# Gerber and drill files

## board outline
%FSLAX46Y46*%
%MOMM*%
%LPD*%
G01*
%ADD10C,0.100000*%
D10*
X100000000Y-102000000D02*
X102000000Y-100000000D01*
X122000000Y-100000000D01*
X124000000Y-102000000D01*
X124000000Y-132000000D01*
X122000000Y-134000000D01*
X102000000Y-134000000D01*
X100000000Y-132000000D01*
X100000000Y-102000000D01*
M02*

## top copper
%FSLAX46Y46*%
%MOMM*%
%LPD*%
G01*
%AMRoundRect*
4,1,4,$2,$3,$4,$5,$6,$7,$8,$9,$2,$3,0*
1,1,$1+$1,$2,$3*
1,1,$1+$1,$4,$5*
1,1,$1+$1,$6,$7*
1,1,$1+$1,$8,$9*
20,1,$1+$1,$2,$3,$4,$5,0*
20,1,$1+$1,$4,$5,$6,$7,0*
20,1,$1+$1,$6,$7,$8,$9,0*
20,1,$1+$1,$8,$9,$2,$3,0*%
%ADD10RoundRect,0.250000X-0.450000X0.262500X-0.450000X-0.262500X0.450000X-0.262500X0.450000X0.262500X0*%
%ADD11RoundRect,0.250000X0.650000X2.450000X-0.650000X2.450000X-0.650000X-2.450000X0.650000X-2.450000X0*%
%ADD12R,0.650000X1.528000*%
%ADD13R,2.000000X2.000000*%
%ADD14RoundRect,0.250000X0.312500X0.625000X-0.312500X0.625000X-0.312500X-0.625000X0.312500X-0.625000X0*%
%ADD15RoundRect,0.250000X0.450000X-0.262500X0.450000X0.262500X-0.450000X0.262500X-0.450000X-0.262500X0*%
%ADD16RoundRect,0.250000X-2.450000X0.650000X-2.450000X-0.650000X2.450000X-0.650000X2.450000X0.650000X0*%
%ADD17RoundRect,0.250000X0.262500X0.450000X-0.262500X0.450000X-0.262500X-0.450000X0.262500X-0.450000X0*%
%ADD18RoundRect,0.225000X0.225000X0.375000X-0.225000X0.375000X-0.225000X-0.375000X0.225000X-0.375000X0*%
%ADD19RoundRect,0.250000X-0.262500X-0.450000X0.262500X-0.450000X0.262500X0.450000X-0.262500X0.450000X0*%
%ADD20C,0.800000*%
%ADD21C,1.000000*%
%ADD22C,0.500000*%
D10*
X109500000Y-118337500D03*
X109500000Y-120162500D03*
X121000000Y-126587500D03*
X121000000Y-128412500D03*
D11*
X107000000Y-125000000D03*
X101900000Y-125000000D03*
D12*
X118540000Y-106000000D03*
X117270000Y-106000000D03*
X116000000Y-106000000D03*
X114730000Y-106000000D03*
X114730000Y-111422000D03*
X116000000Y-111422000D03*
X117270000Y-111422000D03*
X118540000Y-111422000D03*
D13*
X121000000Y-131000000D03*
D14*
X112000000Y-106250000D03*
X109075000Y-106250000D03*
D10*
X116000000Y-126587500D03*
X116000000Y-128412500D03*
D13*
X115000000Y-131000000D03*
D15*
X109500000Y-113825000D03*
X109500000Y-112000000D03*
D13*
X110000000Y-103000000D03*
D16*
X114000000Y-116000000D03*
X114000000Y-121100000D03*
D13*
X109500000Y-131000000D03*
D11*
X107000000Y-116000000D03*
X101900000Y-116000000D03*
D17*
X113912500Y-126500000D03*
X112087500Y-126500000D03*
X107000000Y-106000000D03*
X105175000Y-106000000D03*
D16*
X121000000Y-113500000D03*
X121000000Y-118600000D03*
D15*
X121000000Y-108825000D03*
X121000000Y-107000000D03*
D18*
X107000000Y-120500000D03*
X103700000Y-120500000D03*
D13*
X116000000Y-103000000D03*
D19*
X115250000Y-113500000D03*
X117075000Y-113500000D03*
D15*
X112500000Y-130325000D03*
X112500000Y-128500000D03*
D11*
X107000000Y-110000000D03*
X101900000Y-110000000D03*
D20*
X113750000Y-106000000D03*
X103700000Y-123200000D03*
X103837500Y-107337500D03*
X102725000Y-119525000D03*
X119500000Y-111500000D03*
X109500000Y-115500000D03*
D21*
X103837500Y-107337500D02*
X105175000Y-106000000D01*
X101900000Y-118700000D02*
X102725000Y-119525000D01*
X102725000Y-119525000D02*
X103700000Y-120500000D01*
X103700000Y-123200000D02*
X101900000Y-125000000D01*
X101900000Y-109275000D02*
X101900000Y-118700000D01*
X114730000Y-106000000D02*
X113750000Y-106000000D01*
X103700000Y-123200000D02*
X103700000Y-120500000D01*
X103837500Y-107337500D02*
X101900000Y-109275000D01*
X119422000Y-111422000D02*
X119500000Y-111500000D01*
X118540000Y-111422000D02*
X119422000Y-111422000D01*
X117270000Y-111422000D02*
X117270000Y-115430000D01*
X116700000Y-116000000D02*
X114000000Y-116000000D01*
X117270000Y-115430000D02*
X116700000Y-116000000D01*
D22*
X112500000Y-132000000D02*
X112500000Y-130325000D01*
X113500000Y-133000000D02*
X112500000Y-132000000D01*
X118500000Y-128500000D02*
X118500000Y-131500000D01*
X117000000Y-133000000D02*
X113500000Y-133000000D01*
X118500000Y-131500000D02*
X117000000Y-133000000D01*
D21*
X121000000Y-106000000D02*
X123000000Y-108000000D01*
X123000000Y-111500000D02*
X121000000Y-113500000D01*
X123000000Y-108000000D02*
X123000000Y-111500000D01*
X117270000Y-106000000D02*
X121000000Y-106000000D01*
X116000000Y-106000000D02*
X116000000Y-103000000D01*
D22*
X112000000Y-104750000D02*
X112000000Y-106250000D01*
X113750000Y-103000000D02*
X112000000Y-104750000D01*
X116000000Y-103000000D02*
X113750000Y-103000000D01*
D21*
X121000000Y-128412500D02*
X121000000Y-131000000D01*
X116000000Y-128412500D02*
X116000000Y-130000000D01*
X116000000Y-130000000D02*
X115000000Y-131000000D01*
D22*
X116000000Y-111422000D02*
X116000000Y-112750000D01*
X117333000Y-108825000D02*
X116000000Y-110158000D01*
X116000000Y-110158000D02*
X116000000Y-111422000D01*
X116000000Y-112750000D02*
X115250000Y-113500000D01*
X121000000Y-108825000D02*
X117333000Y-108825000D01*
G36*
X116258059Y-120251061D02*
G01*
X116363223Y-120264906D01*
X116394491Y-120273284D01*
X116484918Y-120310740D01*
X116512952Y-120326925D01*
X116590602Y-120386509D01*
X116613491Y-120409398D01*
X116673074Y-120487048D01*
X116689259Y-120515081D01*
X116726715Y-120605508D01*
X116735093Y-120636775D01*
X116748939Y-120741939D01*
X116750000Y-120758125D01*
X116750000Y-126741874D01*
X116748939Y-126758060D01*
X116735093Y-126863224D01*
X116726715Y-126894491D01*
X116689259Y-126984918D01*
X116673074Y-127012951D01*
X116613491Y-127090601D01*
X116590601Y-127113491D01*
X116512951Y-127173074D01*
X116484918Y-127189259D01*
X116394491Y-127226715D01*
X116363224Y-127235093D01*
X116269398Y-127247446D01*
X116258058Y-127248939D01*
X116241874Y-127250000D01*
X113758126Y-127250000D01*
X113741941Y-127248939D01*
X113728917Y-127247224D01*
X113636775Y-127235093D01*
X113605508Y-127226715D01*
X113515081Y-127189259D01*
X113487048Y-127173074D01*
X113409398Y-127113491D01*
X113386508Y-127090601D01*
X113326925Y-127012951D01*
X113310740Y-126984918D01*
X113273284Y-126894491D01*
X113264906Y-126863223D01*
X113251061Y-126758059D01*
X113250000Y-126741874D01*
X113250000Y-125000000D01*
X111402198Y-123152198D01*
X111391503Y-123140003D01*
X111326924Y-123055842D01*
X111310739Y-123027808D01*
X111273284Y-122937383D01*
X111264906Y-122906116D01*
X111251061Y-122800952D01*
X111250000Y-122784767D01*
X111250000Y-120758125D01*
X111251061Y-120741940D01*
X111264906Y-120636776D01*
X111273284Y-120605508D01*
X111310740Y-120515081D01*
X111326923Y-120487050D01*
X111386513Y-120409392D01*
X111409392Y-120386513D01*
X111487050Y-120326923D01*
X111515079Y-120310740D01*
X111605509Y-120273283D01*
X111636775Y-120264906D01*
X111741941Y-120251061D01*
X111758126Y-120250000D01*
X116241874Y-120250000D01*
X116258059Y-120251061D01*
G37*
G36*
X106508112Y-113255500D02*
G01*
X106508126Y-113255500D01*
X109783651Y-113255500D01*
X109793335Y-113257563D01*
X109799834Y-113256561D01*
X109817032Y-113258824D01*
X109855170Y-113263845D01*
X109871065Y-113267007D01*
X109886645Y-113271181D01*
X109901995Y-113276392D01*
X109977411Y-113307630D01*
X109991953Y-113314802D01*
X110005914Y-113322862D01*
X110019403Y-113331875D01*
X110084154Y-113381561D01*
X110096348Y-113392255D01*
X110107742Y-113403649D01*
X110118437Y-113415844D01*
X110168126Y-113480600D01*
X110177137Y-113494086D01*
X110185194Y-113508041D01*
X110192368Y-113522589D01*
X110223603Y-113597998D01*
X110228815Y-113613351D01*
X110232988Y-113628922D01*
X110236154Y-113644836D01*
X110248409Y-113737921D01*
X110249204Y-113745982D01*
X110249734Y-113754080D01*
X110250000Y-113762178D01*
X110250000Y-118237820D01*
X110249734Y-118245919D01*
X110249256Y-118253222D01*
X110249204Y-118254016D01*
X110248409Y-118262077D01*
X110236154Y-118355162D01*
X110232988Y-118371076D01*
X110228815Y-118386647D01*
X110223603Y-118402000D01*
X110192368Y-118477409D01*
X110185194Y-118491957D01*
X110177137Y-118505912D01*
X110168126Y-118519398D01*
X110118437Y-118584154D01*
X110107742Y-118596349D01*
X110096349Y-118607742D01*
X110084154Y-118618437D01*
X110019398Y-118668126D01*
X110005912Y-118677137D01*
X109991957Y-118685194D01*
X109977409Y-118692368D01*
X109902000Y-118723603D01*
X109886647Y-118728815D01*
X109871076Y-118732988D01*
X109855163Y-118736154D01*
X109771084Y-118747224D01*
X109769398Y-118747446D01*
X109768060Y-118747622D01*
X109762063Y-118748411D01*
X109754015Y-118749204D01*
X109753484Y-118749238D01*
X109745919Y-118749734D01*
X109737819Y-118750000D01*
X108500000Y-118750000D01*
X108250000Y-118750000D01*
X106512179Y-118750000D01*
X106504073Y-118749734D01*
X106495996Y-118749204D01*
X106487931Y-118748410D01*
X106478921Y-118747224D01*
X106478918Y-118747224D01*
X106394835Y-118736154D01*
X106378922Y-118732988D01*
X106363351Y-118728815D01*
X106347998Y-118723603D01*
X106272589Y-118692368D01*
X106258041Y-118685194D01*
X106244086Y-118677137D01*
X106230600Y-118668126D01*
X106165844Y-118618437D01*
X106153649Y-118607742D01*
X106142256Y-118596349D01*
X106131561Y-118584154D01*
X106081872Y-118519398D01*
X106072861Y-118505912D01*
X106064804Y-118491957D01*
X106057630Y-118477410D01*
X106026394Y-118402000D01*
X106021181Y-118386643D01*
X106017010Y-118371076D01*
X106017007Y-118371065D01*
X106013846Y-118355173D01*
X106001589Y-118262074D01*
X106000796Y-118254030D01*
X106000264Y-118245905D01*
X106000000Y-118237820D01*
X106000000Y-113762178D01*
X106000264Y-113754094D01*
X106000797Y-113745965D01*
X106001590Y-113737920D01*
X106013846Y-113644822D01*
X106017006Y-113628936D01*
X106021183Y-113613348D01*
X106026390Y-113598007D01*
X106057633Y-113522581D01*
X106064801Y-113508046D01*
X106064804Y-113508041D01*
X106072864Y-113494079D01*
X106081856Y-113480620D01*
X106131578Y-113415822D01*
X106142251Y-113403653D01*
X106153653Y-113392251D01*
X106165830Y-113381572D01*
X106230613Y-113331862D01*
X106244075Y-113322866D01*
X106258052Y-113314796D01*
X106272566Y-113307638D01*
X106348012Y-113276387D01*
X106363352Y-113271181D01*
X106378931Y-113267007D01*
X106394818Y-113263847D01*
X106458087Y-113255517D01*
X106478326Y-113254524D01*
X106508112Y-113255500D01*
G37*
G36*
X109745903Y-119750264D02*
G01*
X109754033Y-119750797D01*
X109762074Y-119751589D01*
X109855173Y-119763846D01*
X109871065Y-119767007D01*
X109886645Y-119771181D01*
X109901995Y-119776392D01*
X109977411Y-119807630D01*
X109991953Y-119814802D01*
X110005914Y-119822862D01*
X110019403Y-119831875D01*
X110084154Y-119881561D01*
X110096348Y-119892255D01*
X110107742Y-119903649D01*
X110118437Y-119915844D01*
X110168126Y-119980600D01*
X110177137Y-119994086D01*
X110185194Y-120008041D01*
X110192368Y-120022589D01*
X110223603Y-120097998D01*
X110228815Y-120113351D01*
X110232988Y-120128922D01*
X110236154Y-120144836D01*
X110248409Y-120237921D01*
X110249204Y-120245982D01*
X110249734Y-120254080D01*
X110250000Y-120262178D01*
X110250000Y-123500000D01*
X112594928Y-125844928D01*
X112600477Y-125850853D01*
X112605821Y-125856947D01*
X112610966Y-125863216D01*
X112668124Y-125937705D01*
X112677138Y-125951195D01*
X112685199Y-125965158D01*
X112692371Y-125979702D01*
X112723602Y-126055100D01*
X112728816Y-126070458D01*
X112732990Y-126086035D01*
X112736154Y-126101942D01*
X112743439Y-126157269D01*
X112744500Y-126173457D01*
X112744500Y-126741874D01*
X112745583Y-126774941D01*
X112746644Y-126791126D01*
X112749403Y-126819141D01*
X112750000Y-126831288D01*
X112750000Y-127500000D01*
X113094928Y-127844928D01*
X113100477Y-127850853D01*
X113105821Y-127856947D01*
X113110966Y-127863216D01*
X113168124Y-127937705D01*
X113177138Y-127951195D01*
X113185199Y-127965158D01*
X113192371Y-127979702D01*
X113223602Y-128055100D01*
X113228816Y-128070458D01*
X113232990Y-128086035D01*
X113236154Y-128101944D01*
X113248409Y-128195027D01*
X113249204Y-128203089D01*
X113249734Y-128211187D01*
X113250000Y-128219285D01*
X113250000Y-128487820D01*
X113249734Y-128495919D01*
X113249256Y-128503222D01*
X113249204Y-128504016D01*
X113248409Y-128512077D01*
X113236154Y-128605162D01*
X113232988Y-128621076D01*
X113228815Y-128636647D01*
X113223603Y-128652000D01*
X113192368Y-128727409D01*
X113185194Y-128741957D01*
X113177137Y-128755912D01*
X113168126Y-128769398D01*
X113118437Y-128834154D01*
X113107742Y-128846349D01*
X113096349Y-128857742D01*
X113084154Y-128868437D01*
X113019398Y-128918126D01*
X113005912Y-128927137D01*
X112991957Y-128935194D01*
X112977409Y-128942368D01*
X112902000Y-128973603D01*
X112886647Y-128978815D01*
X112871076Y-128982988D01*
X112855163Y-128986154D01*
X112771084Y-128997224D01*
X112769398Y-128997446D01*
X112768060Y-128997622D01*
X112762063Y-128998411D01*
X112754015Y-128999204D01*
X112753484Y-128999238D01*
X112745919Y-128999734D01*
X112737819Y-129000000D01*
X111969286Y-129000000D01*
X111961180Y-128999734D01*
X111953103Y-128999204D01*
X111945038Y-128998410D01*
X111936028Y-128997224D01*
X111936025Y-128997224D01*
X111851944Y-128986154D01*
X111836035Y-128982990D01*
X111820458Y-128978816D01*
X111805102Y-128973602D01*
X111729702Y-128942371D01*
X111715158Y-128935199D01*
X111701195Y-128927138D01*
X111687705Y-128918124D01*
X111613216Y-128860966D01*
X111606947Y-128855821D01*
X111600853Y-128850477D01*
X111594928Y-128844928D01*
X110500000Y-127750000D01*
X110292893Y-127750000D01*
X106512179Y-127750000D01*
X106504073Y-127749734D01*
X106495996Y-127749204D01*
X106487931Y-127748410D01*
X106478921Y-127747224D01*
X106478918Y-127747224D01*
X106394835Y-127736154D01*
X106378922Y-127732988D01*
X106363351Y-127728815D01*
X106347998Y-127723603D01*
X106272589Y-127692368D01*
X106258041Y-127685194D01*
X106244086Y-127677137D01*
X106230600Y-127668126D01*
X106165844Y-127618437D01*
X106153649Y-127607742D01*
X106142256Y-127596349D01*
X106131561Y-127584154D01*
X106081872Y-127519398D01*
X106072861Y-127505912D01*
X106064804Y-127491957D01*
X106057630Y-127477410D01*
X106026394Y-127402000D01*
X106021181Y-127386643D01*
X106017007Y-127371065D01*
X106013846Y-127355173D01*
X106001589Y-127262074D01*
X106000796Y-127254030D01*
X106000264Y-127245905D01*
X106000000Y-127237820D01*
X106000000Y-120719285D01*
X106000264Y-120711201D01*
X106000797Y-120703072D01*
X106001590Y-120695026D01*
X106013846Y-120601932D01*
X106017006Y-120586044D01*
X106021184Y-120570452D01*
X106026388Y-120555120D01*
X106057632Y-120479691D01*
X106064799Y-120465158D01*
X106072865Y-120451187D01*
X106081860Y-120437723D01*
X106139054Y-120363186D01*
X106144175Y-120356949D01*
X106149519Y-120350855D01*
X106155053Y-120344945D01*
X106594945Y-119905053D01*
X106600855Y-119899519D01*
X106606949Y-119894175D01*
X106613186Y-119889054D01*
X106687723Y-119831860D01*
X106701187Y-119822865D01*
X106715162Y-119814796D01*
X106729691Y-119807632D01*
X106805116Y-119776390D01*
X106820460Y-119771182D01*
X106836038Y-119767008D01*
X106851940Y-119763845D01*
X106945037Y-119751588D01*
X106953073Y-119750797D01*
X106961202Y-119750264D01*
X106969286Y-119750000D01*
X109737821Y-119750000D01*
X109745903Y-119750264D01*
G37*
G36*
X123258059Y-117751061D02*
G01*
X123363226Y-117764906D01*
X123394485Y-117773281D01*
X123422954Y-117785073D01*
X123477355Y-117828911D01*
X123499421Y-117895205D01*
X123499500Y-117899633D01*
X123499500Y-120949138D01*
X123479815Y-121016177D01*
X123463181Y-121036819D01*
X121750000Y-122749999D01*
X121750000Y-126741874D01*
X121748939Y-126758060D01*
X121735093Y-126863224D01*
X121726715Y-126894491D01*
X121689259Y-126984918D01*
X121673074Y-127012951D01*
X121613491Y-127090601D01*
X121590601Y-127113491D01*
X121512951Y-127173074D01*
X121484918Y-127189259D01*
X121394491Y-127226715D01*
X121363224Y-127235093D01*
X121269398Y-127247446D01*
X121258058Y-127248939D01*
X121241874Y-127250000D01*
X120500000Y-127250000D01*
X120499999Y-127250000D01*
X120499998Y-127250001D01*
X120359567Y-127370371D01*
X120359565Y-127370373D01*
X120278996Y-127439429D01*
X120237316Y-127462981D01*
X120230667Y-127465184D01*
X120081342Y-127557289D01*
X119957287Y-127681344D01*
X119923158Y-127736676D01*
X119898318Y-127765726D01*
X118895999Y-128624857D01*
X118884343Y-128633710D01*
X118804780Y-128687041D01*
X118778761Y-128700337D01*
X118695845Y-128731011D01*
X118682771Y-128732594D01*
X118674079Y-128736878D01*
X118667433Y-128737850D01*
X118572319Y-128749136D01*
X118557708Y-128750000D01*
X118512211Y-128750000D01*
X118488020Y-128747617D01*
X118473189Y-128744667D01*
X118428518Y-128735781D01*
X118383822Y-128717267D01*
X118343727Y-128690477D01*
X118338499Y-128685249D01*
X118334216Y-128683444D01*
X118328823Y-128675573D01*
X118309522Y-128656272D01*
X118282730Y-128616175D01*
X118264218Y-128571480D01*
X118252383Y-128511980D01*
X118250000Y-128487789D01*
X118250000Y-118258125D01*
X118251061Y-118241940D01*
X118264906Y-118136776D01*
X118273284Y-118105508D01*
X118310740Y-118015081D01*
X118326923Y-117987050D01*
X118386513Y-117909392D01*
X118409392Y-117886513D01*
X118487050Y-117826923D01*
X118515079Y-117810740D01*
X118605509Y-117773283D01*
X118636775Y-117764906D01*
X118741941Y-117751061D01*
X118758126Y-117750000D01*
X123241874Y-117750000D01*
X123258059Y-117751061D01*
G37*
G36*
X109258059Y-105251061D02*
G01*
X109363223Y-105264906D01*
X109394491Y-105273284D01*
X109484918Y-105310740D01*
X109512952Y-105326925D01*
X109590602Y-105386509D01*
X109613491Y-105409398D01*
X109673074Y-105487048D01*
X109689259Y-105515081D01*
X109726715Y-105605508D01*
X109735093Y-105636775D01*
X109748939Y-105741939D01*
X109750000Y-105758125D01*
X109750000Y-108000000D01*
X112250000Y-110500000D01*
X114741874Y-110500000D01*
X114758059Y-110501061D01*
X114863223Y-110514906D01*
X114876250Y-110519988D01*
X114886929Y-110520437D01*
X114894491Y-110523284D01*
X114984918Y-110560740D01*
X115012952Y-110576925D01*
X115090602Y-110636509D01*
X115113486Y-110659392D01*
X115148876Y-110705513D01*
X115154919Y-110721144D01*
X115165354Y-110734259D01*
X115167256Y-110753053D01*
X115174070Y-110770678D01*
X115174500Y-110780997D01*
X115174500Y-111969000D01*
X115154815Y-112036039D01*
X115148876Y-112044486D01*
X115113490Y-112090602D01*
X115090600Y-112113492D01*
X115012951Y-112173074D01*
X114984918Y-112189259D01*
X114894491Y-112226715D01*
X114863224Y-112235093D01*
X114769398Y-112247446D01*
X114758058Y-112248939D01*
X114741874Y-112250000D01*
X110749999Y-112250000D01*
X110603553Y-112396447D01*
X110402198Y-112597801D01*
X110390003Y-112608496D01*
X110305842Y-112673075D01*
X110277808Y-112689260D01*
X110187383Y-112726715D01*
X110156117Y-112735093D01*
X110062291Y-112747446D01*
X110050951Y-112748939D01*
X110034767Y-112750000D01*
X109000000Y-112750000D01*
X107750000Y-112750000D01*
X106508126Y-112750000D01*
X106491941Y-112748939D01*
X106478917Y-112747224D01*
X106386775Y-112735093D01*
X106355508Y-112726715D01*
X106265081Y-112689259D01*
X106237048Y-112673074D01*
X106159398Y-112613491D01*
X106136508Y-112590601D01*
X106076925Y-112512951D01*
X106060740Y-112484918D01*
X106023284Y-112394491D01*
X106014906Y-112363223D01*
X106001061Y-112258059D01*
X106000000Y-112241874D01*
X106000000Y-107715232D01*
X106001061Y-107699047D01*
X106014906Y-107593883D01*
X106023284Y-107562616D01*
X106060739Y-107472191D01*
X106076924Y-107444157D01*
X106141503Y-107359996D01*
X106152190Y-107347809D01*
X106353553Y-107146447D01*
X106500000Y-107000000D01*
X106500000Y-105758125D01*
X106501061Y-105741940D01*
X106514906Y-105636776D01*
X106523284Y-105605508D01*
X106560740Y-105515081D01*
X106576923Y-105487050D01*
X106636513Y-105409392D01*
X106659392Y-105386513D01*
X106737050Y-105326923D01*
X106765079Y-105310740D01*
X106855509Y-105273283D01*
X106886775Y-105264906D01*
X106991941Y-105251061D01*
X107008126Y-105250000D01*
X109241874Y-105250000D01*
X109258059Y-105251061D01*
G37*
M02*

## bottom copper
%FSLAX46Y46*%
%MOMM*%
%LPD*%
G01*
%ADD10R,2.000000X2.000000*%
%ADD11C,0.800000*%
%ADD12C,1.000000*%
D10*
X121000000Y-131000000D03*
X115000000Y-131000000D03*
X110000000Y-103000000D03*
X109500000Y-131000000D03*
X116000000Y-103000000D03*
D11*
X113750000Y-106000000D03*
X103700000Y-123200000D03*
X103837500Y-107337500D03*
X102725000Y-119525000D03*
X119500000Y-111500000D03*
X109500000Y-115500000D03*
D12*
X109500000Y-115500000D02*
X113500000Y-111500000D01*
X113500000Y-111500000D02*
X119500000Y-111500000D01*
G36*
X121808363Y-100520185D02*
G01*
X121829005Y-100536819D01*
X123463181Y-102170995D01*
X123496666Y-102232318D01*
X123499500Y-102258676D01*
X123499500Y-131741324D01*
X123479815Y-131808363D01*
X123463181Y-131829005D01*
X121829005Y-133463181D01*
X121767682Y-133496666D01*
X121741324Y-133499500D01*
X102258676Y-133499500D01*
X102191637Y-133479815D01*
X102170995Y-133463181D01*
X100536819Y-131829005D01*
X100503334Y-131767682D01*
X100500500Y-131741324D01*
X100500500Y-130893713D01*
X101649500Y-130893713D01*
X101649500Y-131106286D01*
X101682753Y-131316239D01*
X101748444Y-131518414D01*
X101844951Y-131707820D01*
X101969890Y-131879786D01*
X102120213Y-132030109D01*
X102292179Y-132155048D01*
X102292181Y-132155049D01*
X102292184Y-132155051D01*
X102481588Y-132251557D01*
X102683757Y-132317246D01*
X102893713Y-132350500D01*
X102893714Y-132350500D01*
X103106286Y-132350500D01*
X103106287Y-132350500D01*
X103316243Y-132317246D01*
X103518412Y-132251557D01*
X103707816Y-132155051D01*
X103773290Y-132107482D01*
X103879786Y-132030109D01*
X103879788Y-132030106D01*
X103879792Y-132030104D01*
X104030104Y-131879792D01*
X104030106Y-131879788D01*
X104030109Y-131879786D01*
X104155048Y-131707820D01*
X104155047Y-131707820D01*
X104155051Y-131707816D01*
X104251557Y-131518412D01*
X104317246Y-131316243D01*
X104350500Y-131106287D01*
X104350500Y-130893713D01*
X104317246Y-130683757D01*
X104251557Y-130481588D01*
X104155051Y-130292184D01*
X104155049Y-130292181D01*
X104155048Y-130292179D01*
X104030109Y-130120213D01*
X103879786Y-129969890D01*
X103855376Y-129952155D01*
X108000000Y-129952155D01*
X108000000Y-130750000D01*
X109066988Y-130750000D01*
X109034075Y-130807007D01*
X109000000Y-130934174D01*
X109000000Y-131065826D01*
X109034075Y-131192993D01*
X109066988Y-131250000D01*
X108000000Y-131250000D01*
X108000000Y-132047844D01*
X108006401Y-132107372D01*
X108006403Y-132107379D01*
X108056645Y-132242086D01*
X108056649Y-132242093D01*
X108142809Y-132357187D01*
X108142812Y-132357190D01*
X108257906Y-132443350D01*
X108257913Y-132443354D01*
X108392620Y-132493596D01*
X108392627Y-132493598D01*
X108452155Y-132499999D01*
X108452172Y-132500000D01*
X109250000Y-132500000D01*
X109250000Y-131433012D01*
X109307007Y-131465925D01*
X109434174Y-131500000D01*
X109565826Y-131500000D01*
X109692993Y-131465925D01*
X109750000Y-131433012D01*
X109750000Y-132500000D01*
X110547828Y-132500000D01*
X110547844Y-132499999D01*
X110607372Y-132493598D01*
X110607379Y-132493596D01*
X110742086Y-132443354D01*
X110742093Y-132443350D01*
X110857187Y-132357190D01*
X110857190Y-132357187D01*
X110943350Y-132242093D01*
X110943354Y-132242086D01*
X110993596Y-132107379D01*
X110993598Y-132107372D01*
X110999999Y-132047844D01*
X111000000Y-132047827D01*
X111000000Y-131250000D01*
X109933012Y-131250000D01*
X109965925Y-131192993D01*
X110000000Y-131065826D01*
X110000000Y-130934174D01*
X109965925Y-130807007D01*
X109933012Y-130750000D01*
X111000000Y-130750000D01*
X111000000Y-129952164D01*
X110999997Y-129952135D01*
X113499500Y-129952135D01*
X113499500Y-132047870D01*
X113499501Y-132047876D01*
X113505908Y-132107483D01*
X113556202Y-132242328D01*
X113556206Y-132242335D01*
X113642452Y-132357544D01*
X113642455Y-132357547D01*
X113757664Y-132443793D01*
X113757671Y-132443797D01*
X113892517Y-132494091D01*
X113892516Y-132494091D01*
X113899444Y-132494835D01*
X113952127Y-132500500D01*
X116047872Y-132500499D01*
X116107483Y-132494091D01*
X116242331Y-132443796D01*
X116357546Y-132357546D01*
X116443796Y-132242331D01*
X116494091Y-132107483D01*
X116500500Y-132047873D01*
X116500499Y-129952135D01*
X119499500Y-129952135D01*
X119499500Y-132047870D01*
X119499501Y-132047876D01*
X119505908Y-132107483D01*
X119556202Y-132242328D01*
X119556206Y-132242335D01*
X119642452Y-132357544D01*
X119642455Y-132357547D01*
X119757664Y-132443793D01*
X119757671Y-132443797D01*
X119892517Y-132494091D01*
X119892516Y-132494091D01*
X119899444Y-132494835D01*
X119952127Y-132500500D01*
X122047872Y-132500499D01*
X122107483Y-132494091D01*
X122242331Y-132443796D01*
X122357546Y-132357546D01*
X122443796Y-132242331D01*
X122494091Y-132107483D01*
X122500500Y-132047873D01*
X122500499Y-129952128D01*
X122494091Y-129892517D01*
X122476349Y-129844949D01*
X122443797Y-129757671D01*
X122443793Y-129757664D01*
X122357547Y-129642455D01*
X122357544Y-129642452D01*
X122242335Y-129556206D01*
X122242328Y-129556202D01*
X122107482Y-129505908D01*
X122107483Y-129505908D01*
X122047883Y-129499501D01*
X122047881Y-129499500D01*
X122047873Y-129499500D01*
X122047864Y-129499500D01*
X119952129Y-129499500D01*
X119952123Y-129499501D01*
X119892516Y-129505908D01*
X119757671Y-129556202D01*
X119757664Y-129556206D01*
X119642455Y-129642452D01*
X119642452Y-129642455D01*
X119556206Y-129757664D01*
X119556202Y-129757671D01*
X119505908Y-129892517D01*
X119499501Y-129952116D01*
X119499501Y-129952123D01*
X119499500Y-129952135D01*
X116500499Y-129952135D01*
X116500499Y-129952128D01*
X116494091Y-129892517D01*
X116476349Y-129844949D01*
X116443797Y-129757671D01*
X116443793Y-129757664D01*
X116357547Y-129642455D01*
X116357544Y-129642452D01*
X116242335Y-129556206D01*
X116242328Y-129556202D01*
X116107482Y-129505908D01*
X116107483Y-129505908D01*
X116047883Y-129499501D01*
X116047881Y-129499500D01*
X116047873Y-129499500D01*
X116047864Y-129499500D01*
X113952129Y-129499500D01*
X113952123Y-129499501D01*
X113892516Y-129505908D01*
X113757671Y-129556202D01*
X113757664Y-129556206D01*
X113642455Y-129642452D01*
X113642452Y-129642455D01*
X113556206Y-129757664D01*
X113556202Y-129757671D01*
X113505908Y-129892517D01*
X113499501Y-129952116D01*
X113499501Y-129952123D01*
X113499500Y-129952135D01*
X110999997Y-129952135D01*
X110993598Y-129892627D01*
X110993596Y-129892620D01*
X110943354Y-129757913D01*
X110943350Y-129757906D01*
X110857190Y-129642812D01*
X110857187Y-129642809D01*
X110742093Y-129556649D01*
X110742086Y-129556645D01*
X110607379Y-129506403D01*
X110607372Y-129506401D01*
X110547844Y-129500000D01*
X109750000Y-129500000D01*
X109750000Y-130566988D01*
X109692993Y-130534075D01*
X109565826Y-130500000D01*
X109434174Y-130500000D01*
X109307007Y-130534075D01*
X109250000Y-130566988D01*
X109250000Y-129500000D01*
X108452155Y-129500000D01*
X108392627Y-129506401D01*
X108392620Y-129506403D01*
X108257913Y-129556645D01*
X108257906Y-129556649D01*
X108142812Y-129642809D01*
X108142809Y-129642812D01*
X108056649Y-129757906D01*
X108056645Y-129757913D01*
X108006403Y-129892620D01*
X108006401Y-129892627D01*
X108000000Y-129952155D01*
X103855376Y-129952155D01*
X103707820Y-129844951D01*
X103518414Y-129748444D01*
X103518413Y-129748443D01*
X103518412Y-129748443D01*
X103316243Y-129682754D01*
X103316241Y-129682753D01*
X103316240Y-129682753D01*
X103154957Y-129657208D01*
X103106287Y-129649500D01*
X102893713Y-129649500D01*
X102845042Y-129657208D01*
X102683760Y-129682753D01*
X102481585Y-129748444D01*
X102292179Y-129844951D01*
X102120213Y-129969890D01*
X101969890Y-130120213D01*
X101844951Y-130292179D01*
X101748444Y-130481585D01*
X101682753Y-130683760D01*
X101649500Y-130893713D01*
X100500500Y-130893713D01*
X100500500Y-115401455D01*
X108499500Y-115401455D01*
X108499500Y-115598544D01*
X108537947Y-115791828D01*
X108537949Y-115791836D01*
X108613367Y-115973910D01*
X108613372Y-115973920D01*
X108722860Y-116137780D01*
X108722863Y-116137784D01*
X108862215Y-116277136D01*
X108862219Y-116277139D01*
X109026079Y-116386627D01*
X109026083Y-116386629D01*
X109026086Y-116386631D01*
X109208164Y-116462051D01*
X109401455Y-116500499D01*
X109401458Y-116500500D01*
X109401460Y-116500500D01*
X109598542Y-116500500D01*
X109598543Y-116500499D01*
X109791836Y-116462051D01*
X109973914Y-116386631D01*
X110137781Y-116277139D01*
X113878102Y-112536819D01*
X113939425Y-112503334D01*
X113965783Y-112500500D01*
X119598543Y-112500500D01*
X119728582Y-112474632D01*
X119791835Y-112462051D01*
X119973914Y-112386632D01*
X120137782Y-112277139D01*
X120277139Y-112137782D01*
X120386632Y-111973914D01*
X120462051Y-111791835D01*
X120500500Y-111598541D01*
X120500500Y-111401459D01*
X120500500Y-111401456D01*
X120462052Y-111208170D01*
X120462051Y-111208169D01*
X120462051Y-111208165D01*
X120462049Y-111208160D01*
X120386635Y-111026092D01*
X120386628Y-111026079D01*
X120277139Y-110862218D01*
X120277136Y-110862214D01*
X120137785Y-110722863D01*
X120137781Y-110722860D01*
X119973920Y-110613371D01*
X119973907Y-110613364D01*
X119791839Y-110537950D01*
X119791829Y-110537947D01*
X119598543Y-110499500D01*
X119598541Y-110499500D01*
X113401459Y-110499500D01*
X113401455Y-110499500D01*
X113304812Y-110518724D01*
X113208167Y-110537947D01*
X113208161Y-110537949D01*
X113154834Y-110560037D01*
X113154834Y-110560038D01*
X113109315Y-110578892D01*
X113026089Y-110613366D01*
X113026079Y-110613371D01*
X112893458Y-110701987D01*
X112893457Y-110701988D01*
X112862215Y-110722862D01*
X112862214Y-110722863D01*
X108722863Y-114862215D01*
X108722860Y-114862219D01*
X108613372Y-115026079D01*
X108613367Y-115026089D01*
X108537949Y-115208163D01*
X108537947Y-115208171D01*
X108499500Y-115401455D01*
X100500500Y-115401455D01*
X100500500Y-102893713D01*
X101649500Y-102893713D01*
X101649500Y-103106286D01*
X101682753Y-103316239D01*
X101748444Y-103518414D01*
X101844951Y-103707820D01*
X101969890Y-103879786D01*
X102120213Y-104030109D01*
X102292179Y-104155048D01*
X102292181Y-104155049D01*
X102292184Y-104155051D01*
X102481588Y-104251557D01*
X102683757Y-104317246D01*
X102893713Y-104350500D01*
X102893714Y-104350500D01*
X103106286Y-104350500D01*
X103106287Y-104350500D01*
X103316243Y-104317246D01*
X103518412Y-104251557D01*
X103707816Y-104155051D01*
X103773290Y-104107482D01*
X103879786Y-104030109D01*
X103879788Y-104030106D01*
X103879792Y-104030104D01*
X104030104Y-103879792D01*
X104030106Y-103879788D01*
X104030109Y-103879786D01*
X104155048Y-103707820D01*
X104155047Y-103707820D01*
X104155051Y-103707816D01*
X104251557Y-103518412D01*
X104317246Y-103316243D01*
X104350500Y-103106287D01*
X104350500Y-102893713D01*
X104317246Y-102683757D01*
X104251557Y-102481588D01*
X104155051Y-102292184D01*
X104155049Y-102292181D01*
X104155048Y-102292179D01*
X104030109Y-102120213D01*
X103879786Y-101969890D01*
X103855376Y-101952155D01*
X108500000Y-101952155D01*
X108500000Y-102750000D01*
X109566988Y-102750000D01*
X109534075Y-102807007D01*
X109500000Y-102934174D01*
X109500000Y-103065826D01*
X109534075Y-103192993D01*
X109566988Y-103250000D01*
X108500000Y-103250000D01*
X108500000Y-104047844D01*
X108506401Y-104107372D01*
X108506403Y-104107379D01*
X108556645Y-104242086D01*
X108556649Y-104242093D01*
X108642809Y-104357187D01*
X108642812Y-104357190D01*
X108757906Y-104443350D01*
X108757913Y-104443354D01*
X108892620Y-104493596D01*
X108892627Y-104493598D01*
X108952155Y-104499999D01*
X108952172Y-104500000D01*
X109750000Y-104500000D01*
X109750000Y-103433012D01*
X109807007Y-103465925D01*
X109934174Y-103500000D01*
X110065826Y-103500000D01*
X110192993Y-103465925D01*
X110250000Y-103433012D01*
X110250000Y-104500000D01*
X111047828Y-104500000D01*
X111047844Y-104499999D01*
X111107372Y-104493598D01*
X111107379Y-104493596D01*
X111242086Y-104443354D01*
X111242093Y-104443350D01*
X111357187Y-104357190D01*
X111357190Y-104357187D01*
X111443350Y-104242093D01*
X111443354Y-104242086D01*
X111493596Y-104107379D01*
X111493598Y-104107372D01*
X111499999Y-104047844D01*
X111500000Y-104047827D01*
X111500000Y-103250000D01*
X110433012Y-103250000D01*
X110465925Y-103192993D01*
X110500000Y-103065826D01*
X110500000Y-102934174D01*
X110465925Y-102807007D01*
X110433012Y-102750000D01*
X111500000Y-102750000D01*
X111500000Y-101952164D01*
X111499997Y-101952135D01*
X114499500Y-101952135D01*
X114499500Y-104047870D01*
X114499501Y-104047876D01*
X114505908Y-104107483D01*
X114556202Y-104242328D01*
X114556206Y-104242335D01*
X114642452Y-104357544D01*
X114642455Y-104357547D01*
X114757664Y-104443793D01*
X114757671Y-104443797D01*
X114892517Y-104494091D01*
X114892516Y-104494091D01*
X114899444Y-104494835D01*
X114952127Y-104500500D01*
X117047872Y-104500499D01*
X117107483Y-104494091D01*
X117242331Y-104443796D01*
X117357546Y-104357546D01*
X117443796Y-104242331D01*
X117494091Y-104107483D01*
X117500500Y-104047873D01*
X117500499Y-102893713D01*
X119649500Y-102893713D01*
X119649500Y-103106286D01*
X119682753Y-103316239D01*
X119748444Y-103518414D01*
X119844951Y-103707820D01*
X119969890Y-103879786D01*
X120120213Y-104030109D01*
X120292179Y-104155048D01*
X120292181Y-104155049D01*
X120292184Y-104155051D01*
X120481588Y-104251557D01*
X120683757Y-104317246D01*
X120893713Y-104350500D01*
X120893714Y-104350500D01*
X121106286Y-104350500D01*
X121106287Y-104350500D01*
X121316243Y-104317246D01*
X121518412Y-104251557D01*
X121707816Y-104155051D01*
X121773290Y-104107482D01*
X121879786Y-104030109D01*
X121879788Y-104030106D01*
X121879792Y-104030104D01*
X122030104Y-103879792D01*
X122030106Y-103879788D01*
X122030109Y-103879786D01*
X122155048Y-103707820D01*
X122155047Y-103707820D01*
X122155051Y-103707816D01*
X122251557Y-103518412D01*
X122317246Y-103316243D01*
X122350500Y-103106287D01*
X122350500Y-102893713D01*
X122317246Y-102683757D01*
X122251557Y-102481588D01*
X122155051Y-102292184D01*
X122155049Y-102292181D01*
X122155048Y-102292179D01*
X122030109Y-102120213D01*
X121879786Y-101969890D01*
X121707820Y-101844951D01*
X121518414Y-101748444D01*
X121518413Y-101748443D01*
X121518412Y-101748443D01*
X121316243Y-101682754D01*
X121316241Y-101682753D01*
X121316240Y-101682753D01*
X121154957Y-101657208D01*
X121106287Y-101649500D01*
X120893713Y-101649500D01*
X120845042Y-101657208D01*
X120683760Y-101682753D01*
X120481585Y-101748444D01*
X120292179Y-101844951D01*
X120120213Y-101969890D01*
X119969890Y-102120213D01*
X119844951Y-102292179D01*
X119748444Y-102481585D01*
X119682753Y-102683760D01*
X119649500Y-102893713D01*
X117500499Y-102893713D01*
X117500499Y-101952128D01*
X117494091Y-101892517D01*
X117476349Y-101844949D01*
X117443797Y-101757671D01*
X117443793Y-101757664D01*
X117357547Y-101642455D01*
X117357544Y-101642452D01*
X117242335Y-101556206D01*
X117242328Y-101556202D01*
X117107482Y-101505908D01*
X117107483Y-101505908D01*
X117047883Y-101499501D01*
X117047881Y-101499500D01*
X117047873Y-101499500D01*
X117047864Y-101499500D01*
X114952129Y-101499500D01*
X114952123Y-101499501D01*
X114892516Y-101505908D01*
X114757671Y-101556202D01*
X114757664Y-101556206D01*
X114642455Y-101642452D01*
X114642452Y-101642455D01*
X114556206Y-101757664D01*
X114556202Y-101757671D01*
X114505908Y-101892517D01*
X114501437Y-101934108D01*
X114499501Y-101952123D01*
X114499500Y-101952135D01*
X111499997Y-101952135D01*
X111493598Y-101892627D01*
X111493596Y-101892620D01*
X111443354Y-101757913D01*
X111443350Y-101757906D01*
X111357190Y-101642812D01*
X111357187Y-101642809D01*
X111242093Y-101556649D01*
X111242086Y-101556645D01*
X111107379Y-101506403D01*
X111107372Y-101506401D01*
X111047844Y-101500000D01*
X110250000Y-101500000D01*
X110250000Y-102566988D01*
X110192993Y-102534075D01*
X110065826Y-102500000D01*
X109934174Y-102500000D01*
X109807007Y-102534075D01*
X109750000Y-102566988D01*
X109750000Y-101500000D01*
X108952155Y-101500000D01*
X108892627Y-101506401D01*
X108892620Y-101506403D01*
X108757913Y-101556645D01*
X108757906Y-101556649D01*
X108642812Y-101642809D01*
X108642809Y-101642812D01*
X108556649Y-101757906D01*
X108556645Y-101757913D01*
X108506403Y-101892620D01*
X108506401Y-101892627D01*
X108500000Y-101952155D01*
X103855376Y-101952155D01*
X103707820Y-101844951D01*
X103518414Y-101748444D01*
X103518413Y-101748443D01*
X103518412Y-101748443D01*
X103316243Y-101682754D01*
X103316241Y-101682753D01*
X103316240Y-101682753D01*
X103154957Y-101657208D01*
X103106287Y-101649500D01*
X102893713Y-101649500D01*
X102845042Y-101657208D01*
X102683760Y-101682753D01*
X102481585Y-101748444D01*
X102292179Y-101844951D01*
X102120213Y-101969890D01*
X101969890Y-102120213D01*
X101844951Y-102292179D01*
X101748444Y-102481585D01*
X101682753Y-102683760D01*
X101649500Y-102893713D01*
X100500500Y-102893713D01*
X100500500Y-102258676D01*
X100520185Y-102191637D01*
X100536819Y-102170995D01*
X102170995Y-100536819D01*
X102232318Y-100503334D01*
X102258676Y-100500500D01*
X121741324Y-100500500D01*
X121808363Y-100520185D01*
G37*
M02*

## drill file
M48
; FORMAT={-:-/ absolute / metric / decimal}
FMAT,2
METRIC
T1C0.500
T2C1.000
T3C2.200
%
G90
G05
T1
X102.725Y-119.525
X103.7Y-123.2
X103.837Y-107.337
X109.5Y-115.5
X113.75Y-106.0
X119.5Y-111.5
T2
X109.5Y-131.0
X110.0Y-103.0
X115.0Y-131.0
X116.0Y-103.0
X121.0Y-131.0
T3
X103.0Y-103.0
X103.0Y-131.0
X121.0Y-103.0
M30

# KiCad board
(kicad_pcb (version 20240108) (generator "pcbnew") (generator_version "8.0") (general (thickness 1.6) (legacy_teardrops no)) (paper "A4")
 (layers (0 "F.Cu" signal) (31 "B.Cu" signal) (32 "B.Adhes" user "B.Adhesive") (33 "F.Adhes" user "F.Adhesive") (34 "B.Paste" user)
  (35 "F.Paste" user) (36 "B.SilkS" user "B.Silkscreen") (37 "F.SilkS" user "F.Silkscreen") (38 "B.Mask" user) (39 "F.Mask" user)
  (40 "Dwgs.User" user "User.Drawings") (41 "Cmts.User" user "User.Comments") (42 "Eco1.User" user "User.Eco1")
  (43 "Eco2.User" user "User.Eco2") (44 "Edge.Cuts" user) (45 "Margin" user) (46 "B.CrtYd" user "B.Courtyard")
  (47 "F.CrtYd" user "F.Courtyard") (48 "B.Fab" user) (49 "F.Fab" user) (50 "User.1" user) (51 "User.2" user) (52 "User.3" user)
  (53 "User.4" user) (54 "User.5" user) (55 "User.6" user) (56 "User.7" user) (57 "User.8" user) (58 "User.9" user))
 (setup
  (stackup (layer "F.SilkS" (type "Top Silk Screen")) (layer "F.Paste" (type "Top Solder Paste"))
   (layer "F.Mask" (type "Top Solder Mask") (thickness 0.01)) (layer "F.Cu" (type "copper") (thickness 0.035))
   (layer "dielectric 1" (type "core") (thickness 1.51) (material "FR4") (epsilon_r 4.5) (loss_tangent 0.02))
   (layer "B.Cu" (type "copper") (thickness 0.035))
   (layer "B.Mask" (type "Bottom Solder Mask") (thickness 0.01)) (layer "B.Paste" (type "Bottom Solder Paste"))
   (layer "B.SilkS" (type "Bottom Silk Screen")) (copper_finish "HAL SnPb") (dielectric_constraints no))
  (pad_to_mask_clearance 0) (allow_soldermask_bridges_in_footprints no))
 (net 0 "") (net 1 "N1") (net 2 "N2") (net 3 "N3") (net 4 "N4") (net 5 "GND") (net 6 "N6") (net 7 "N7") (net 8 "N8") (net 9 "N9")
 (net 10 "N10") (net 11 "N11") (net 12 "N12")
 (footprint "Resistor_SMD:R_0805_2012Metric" (layer "F.Cu") (at 109.5 119.25 -90)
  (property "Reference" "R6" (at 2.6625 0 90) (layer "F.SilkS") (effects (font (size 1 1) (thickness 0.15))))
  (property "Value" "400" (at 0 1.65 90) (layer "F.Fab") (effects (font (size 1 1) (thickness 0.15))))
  (pad "1" smd roundrect (at -0.9125 0 270) (size 1.025 1.4) (layers "F.Cu" "F.Paste" "F.Mask") (roundrect_rratio 0.243902) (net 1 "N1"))
  (pad "2" smd roundrect (at 0.9125 0 270) (size 1.025 1.4) (layers "F.Cu" "F.Paste" "F.Mask") (roundrect_rratio 0.243902) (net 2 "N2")))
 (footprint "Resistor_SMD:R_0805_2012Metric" (layer "F.Cu") (at 121 127.5 -90)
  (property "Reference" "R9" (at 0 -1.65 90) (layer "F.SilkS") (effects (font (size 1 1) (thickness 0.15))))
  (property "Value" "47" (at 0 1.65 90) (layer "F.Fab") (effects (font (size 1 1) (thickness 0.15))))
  (pad "1" smd roundrect (at -0.9125 0 270) (size 1.025 1.4) (layers "F.Cu" "F.Paste" "F.Mask") (roundrect_rratio 0.243902) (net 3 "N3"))
  (pad "2" smd roundrect (at 0.9125 0 270) (size 1.025 1.4) (layers "F.Cu" "F.Paste" "F.Mask") (roundrect_rratio 0.243902) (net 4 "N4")))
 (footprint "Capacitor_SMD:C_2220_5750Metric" (layer "F.Cu") (at 104.45 125 180)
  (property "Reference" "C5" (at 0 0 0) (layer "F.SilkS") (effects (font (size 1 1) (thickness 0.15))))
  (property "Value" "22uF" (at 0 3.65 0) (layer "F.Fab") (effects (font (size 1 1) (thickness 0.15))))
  (pad "1" smd roundrect (at -2.55 0 180) (size 1.8 5.4) (layers "F.Cu" "F.Paste" "F.Mask") (roundrect_rratio 0.138889) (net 2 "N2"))
  (pad "2" smd roundrect (at 2.55 0 180) (size 1.8 5.4) (layers "F.Cu" "F.Paste" "F.Mask") (roundrect_rratio 0.138889) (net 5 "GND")))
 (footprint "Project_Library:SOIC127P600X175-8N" (layer "F.Cu") (at 116.635 108.711 -90)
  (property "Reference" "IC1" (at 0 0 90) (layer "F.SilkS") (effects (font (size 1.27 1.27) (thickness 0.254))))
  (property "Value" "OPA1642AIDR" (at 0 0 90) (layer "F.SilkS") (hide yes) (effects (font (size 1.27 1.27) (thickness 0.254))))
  (pad "1" smd rect (at -2.711 -1.905) (size 0.65 1.528) (layers "F.Cu" "F.Paste" "F.Mask") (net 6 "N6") (thermal_bridge_angle 45))
  (pad "2" smd rect (at -2.711 -0.635) (size 0.65 1.528) (layers "F.Cu" "F.Paste" "F.Mask") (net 6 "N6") (thermal_bridge_angle 45))
  (pad "3" smd rect (at -2.711 0.635) (size 0.65 1.528) (layers "F.Cu" "F.Paste" "F.Mask") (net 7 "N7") (thermal_bridge_angle 45))
  (pad "4" smd rect (at -2.711 1.905) (size 0.65 1.528) (layers "F.Cu" "F.Paste" "F.Mask") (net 5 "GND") (thermal_bridge_angle 45))
  (pad "5" smd rect (at 2.711 1.905) (size 0.65 1.528) (layers "F.Cu" "F.Paste" "F.Mask") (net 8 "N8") (thermal_bridge_angle 45))
  (pad "6" smd rect (at 2.711 0.635) (size 0.65 1.528) (layers "F.Cu" "F.Paste" "F.Mask") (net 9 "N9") (thermal_bridge_angle 45))
  (pad "7" smd rect (at 2.711 -0.635) (size 0.65 1.528) (layers "F.Cu" "F.Paste" "F.Mask") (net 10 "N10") (thermal_bridge_angle 45))
  (pad "8" smd rect (at 2.711 -1.905) (size 0.65 1.528) (layers "F.Cu" "F.Paste" "F.Mask") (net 1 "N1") (thermal_bridge_angle 45)))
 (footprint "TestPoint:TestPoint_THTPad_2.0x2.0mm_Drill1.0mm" (layer "F.Cu") (at 121 131)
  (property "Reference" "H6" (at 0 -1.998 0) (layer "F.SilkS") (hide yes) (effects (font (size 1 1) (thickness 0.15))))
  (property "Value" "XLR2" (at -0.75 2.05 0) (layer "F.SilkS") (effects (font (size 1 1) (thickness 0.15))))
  (pad "1" thru_hole rect (at 0 0) (size 2 2) (drill 1) (layers "*.Cu" "*.Mask") (remove_unused_layers no) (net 4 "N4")))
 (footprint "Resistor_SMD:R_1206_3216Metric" (layer "F.Cu") (at 110.5375 106.25 180)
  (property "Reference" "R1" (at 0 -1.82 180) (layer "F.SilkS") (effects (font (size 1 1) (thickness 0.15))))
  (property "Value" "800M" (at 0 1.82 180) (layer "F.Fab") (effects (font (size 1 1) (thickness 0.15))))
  (pad "1" smd roundrect (at -1.4625 0 180) (size 1.125 1.75) (layers "F.Cu" "F.Paste" "F.Mask") (roundrect_rratio 0.222222) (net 7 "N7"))
  (pad "2" smd roundrect (at 1.4625 0 180) (size 1.125 1.75) (layers "F.Cu" "F.Paste" "F.Mask") (roundrect_rratio 0.222222) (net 8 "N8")))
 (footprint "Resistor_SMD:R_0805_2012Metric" (layer "F.Cu") (at 116 127.5 -90)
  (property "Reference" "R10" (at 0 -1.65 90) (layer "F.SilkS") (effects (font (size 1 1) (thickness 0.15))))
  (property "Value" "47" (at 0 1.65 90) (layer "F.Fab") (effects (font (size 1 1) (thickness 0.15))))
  (pad "1" smd roundrect (at -0.9125 0 270) (size 1.025 1.4) (layers "F.Cu" "F.Paste" "F.Mask") (roundrect_rratio 0.243902) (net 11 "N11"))
  (pad "2" smd roundrect (at 0.9125 0 270) (size 1.025 1.4) (layers "F.Cu" "F.Paste" "F.Mask") (roundrect_rratio 0.243902) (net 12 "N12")))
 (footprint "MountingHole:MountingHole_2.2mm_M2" (layer "F.Cu") (at 103 103)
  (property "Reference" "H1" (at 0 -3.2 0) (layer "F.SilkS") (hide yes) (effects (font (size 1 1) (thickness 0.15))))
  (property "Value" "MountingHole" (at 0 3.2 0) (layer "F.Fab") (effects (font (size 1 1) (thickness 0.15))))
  (pad "" np_thru_hole circle (at 0 0) (size 2.2 2.2) (drill 2.2) (layers "*.Cu" "*.Mask")))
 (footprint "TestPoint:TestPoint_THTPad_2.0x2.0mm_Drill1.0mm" (layer "F.Cu") (at 115 131)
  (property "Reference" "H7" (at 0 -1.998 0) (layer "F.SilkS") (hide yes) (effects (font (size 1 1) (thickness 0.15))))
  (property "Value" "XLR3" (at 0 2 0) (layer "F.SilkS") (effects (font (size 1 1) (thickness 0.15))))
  (pad "1" thru_hole rect (at 0 0) (size 2 2) (drill 1) (layers "*.Cu" "*.Mask") (remove_unused_layers no) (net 12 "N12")))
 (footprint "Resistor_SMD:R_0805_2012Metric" (layer "F.Cu") (at 109.5 112.9125 90)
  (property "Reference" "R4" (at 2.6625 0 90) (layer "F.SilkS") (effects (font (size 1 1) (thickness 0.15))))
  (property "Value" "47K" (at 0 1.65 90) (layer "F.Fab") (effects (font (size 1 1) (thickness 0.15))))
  (pad "1" smd roundrect (at -0.9125 0 90) (size 1.025 1.4) (layers "F.Cu" "F.Paste" "F.Mask") (roundrect_rratio 0.243902) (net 1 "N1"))
  (pad "2" smd roundrect (at 0.9125 0 90) (size 1.025 1.4) (layers "F.Cu" "F.Paste" "F.Mask") (roundrect_rratio 0.243902) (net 8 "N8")))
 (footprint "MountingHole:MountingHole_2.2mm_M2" (layer "F.Cu") (at 103 131)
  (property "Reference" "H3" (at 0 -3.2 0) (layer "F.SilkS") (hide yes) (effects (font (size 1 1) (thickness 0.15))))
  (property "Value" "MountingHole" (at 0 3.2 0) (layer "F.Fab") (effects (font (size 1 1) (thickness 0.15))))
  (pad "" np_thru_hole circle (at 0 0) (size 2.2 2.2) (drill 2.2) (layers "*.Cu" "*.Mask")))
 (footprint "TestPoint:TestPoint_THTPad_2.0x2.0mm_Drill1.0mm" (layer "F.Cu") (at 110 103)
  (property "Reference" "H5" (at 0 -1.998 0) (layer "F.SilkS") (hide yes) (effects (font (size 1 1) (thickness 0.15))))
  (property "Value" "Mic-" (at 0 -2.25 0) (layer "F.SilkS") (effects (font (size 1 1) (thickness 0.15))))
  (pad "1" thru_hole rect (at 0 0) (size 2 2) (drill 1) (layers "*.Cu" "*.Mask") (remove_unused_layers no) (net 5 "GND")))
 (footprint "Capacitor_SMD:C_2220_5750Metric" (layer "F.Cu") (at 114 118.55 -90)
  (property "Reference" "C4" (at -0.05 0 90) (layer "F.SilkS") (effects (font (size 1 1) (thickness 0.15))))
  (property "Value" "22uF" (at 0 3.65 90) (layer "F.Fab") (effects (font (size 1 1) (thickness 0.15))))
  (pad "1" smd roundrect (at -2.55 0 270) (size 1.8 5.4) (layers "F.Cu" "F.Paste" "F.Mask") (roundrect_rratio 0.138889) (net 10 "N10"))
  (pad "2" smd roundrect (at 2.55 0 270) (size 1.8 5.4) (layers "F.Cu" "F.Paste" "F.Mask") (roundrect_rratio 0.138889) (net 11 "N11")))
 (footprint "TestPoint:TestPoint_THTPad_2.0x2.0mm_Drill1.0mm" (layer "F.Cu") (at 109.5 131)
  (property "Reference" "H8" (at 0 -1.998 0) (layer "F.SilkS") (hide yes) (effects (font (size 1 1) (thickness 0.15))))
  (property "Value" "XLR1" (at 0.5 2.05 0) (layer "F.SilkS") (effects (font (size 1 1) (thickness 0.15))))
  (pad "1" thru_hole rect (at 0 0) (size 2 2) (drill 1) (layers "*.Cu" "*.Mask") (remove_unused_layers no) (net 5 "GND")))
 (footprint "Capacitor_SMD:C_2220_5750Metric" (layer "F.Cu") (at 104.45 116 180)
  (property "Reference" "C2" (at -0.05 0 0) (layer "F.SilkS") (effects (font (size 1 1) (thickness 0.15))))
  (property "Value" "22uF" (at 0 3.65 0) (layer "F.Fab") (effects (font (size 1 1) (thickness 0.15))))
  (pad "1" smd roundrect (at -2.55 0 180) (size 1.8 5.4) (layers "F.Cu" "F.Paste" "F.Mask") (roundrect_rratio 0.138889) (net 1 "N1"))
  (pad "2" smd roundrect (at 2.55 0 180) (size 1.8 5.4) (layers "F.Cu" "F.Paste" "F.Mask") (roundrect_rratio 0.138889) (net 5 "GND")))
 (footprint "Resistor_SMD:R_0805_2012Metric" (layer "F.Cu") (at 113 126.5 180)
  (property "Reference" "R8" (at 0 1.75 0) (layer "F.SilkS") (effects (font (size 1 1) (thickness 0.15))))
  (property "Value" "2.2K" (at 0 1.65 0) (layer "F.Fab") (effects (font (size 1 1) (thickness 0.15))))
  (pad "1" smd roundrect (at -0.9125 0 180) (size 1.025 1.4) (layers "F.Cu" "F.Paste" "F.Mask") (roundrect_rratio 0.243902) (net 11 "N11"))
  (pad "2" smd roundrect (at 0.9125 0 180) (size 1.025 1.4) (layers "F.Cu" "F.Paste" "F.Mask") (roundrect_rratio 0.243902) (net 2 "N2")))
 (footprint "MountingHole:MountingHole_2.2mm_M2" (layer "F.Cu") (at 121 103)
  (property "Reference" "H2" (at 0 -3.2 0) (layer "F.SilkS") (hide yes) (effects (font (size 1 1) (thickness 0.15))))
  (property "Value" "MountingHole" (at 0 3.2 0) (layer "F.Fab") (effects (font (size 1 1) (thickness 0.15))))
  (pad "" np_thru_hole circle (at 0 0) (size 2.2 2.2) (drill 2.2) (layers "*.Cu" "*.Mask")))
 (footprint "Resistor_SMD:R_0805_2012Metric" (layer "F.Cu") (at 106.0875 106 180)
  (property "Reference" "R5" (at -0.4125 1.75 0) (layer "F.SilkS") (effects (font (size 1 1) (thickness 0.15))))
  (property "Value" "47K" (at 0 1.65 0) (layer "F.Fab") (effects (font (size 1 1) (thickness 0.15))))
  (pad "1" smd roundrect (at -0.9125 0 180) (size 1.025 1.4) (layers "F.Cu" "F.Paste" "F.Mask") (roundrect_rratio 0.243902) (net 8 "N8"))
  (pad "2" smd roundrect (at 0.9125 0 180) (size 1.025 1.4) (layers "F.Cu" "F.Paste" "F.Mask") (roundrect_rratio 0.243902) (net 5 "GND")))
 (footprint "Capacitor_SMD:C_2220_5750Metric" (layer "F.Cu") (at 121 116.05 -90)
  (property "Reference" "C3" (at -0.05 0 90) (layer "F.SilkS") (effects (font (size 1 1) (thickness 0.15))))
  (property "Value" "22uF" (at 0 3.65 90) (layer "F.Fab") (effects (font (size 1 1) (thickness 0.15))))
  (pad "1" smd roundrect (at -2.55 0 270) (size 1.8 5.4) (layers "F.Cu" "F.Paste" "F.Mask") (roundrect_rratio 0.138889) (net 6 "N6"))
  (pad "2" smd roundrect (at 2.55 0 270) (size 1.8 5.4) (layers "F.Cu" "F.Paste" "F.Mask") (roundrect_rratio 0.138889) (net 3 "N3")))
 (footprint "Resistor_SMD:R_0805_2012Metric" (layer "F.Cu") (at 121 107.9125 90)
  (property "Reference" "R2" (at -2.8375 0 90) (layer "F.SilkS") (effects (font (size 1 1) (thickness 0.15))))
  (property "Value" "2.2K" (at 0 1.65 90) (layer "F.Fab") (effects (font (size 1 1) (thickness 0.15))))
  (pad "1" smd roundrect (at -0.9125 0 90) (size 1.025 1.4) (layers "F.Cu" "F.Paste" "F.Mask") (roundrect_rratio 0.243902) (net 9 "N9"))
  (pad "2" smd roundrect (at 0.9125 0 90) (size 1.025 1.4) (layers "F.Cu" "F.Paste" "F.Mask") (roundrect_rratio 0.243902) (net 6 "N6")))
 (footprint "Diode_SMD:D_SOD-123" (layer "F.Cu") (at 105.35 120.5 180)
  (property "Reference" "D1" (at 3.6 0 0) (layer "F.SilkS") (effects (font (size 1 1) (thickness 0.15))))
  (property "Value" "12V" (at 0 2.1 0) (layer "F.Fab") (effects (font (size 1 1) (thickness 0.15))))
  (pad "1" smd roundrect (at -1.65 0 180) (size 0.9 1.2) (layers "F.Cu" "F.Paste" "F.Mask") (roundrect_rratio 0.25) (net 2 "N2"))
  (pad "2" smd roundrect (at 1.65 0 180) (size 0.9 1.2) (layers "F.Cu" "F.Paste" "F.Mask") (roundrect_rratio 0.25) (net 5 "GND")))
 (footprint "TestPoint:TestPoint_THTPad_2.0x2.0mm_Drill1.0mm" (layer "F.Cu") (at 116 103)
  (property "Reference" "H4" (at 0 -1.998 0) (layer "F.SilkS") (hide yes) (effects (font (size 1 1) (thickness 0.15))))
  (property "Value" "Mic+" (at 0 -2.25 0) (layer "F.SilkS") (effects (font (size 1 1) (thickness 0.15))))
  (pad "1" thru_hole rect (at 0 0) (size 2 2) (drill 1) (layers "*.Cu" "*.Mask") (remove_unused_layers no) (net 7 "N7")))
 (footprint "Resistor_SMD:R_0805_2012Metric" (layer "F.Cu") (at 116.1625 113.5)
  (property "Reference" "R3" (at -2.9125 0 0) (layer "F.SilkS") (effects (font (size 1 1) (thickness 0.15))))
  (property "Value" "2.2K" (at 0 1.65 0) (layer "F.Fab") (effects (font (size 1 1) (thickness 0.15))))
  (pad "1" smd roundrect (at -0.9125 0) (size 1.025 1.4) (layers "F.Cu" "F.Paste" "F.Mask") (roundrect_rratio 0.243902) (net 9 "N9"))
  (pad "2" smd roundrect (at 0.9125 0) (size 1.025 1.4) (layers "F.Cu" "F.Paste" "F.Mask") (roundrect_rratio 0.243902) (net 10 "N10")))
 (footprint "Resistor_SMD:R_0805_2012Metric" (layer "F.Cu") (at 112.5 129.4125 90)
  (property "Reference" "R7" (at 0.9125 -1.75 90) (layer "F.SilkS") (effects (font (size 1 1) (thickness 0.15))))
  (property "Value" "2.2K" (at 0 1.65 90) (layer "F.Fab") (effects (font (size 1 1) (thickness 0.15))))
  (pad "1" smd roundrect (at -0.9125 0 90) (size 1.025 1.4) (layers "F.Cu" "F.Paste" "F.Mask") (roundrect_rratio 0.243902) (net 3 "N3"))
  (pad "2" smd roundrect (at 0.9125 0 90) (size 1.025 1.4) (layers "F.Cu" "F.Paste" "F.Mask") (roundrect_rratio 0.243902) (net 2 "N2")))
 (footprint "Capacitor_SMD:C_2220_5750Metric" (layer "F.Cu") (at 104.45 110 180)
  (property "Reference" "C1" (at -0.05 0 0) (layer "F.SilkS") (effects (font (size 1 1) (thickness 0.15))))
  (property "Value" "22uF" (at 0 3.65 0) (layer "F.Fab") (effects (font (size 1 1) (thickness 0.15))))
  (pad "1" smd roundrect (at -2.55 0 180) (size 1.8 5.4) (layers "F.Cu" "F.Paste" "F.Mask") (roundrect_rratio 0.138889) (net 8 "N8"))
  (pad "2" smd roundrect (at 2.55 0 180) (size 1.8 5.4) (layers "F.Cu" "F.Paste" "F.Mask") (roundrect_rratio 0.138889) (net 5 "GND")))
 (gr_poly
  (pts (xy 100 102) (xy 102 100) (xy 122 100) (xy 124 102) (xy 124 132) (xy 122 134) (xy 102 134) (xy 100 132))
  (stroke (width 0.1) (type solid)) (fill none) (layer "Edge.Cuts"))
 (segment (start 103.8375 107.3375) (end 105.175 106) (width 1) (layer "F.Cu") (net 5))
 (segment (start 101.9 118.7) (end 102.725 119.525) (width 1) (layer "F.Cu") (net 5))
 (segment (start 102.725 119.525) (end 103.7 120.5) (width 1) (layer "F.Cu") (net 5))
 (segment (start 103.7 123.2) (end 101.9 125) (width 1) (layer "F.Cu") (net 5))
 (segment (start 101.9 109.275) (end 101.9 118.7) (width 1) (layer "F.Cu") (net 5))
 (segment (start 114.73 106) (end 113.75 106) (width 1) (layer "F.Cu") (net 5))
 (segment (start 103.7 123.2) (end 103.7 120.5) (width 1) (layer "F.Cu") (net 5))
 (segment (start 103.8375 107.3375) (end 101.9 109.275) (width 1) (layer "F.Cu") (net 5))
 (via (at 113.75 106) (size 0.8) (drill 0.5) (layers "F.Cu" "B.Cu") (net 5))
 (via (at 103.7 123.2) (size 0.8) (drill 0.5) (layers "F.Cu" "B.Cu") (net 5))
 (via (at 103.8375 107.3375) (size 0.8) (drill 0.5) (layers "F.Cu" "B.Cu") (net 5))
 (via (at 102.725 119.525) (size 0.8) (drill 0.5) (layers "F.Cu" "B.Cu") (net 5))
 (segment (start 119.422 111.422) (end 119.5 111.5) (width 1) (layer "F.Cu") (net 1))
 (segment (start 118.54 111.422) (end 119.422 111.422) (width 1) (layer "F.Cu") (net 1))
 (via (at 119.5 111.5) (size 0.8) (drill 0.5) (layers "F.Cu" "B.Cu") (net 1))
 (via (at 109.5 115.5) (size 0.8) (drill 0.5) (layers "F.Cu" "B.Cu") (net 1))
 (segment (start 109.5 115.5) (end 113.5 111.5) (width 1) (layer "B.Cu") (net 1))
 (segment (start 113.5 111.5) (end 119.5 111.5) (width 1) (layer "B.Cu") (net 1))
 (segment (start 117.27 111.422) (end 117.27 115.43) (width 1) (layer "F.Cu") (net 10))
 (segment (start 116.7 116) (end 114 116) (width 1) (layer "F.Cu") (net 10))
 (segment (start 117.27 115.43) (end 116.7 116) (width 1) (layer "F.Cu") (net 10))
 (segment (start 112.5 132) (end 112.5 130.325) (width 0.5) (layer "F.Cu") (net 3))
 (segment (start 113.5 133) (end 112.5 132) (width 0.5) (layer "F.Cu") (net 3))
 (segment (start 118.5 128.5) (end 118.5 131.5) (width 0.5) (layer "F.Cu") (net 3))
 (segment (start 117 133) (end 113.5 133) (width 0.5) (layer "F.Cu") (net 3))
 (segment (start 118.5 131.5) (end 117 133) (width 0.5) (layer "F.Cu") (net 3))
 (segment (start 121 106) (end 123 108) (width 1) (layer "F.Cu") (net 6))
 (segment (start 123 111.5) (end 121 113.5) (width 1) (layer "F.Cu") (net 6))
 (segment (start 123 108) (end 123 111.5) (width 1) (layer "F.Cu") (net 6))
 (segment (start 117.27 106) (end 121 106) (width 1) (layer "F.Cu") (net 6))
 (segment (start 116 106) (end 116 103) (width 1) (layer "F.Cu") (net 7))
 (segment (start 112 104.75) (end 112 106.25) (width 0.5) (layer "F.Cu") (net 7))
 (segment (start 113.75 103) (end 112 104.75) (width 0.5) (layer "F.Cu") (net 7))
 (segment (start 116 103) (end 113.75 103) (width 0.5) (layer "F.Cu") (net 7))
 (segment (start 121 128.4125) (end 121 131) (width 1) (layer "F.Cu") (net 4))
 (segment (start 116 128.4125) (end 116 130) (width 1) (layer "F.Cu") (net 12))
 (segment (start 116 130) (end 115 131) (width 1) (layer "F.Cu") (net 12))
 (segment (start 116 111.422) (end 116 112.75) (width 0.5) (layer "F.Cu") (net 9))
 (segment (start 117.333 108.825) (end 116 110.158) (width 0.5) (layer "F.Cu") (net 9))
 (segment (start 116 110.158) (end 116 111.422) (width 0.5) (layer "F.Cu") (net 9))
 (segment (start 116 112.75) (end 115.25 113.5) (width 0.5) (layer "F.Cu") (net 9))
 (segment (start 121 108.825) (end 117.333 108.825) (width 0.5) (layer "F.Cu") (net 9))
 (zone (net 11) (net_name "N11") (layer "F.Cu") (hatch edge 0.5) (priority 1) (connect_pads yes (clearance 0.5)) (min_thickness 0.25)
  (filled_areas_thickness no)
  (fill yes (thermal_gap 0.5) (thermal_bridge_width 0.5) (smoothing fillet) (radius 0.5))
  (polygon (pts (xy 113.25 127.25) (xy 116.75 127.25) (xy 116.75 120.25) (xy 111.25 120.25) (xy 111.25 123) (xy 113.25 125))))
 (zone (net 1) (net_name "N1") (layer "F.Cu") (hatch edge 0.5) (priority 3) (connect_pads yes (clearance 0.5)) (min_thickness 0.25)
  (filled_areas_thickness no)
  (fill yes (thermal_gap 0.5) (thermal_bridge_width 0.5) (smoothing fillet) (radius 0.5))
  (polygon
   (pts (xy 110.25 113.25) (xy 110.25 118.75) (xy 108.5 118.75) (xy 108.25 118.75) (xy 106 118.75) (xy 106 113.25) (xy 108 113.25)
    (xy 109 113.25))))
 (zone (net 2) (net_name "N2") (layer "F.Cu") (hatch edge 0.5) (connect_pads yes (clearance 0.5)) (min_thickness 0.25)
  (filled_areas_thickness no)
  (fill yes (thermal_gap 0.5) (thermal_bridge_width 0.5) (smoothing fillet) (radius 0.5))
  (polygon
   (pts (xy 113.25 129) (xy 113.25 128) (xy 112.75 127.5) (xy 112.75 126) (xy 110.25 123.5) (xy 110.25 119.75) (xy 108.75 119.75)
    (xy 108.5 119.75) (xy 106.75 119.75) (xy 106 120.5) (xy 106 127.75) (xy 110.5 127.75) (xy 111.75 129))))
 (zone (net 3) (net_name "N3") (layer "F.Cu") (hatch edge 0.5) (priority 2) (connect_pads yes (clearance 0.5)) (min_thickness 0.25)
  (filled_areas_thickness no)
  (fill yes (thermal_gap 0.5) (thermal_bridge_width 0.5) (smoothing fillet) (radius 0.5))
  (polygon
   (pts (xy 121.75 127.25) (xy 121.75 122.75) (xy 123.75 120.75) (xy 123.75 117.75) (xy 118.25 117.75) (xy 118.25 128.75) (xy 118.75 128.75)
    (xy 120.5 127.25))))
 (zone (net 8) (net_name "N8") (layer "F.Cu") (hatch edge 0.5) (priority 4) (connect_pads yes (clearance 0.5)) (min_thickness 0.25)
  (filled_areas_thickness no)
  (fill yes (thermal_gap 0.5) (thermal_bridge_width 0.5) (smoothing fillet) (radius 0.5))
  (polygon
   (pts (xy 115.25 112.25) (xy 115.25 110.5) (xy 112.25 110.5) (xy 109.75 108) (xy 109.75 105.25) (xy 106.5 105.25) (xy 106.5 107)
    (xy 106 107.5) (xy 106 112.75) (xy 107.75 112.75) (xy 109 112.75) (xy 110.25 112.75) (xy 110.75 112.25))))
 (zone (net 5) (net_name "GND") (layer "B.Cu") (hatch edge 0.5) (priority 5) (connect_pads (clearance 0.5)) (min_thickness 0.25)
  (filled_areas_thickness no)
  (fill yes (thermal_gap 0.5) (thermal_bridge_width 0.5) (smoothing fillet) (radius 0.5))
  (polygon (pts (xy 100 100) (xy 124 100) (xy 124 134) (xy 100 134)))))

